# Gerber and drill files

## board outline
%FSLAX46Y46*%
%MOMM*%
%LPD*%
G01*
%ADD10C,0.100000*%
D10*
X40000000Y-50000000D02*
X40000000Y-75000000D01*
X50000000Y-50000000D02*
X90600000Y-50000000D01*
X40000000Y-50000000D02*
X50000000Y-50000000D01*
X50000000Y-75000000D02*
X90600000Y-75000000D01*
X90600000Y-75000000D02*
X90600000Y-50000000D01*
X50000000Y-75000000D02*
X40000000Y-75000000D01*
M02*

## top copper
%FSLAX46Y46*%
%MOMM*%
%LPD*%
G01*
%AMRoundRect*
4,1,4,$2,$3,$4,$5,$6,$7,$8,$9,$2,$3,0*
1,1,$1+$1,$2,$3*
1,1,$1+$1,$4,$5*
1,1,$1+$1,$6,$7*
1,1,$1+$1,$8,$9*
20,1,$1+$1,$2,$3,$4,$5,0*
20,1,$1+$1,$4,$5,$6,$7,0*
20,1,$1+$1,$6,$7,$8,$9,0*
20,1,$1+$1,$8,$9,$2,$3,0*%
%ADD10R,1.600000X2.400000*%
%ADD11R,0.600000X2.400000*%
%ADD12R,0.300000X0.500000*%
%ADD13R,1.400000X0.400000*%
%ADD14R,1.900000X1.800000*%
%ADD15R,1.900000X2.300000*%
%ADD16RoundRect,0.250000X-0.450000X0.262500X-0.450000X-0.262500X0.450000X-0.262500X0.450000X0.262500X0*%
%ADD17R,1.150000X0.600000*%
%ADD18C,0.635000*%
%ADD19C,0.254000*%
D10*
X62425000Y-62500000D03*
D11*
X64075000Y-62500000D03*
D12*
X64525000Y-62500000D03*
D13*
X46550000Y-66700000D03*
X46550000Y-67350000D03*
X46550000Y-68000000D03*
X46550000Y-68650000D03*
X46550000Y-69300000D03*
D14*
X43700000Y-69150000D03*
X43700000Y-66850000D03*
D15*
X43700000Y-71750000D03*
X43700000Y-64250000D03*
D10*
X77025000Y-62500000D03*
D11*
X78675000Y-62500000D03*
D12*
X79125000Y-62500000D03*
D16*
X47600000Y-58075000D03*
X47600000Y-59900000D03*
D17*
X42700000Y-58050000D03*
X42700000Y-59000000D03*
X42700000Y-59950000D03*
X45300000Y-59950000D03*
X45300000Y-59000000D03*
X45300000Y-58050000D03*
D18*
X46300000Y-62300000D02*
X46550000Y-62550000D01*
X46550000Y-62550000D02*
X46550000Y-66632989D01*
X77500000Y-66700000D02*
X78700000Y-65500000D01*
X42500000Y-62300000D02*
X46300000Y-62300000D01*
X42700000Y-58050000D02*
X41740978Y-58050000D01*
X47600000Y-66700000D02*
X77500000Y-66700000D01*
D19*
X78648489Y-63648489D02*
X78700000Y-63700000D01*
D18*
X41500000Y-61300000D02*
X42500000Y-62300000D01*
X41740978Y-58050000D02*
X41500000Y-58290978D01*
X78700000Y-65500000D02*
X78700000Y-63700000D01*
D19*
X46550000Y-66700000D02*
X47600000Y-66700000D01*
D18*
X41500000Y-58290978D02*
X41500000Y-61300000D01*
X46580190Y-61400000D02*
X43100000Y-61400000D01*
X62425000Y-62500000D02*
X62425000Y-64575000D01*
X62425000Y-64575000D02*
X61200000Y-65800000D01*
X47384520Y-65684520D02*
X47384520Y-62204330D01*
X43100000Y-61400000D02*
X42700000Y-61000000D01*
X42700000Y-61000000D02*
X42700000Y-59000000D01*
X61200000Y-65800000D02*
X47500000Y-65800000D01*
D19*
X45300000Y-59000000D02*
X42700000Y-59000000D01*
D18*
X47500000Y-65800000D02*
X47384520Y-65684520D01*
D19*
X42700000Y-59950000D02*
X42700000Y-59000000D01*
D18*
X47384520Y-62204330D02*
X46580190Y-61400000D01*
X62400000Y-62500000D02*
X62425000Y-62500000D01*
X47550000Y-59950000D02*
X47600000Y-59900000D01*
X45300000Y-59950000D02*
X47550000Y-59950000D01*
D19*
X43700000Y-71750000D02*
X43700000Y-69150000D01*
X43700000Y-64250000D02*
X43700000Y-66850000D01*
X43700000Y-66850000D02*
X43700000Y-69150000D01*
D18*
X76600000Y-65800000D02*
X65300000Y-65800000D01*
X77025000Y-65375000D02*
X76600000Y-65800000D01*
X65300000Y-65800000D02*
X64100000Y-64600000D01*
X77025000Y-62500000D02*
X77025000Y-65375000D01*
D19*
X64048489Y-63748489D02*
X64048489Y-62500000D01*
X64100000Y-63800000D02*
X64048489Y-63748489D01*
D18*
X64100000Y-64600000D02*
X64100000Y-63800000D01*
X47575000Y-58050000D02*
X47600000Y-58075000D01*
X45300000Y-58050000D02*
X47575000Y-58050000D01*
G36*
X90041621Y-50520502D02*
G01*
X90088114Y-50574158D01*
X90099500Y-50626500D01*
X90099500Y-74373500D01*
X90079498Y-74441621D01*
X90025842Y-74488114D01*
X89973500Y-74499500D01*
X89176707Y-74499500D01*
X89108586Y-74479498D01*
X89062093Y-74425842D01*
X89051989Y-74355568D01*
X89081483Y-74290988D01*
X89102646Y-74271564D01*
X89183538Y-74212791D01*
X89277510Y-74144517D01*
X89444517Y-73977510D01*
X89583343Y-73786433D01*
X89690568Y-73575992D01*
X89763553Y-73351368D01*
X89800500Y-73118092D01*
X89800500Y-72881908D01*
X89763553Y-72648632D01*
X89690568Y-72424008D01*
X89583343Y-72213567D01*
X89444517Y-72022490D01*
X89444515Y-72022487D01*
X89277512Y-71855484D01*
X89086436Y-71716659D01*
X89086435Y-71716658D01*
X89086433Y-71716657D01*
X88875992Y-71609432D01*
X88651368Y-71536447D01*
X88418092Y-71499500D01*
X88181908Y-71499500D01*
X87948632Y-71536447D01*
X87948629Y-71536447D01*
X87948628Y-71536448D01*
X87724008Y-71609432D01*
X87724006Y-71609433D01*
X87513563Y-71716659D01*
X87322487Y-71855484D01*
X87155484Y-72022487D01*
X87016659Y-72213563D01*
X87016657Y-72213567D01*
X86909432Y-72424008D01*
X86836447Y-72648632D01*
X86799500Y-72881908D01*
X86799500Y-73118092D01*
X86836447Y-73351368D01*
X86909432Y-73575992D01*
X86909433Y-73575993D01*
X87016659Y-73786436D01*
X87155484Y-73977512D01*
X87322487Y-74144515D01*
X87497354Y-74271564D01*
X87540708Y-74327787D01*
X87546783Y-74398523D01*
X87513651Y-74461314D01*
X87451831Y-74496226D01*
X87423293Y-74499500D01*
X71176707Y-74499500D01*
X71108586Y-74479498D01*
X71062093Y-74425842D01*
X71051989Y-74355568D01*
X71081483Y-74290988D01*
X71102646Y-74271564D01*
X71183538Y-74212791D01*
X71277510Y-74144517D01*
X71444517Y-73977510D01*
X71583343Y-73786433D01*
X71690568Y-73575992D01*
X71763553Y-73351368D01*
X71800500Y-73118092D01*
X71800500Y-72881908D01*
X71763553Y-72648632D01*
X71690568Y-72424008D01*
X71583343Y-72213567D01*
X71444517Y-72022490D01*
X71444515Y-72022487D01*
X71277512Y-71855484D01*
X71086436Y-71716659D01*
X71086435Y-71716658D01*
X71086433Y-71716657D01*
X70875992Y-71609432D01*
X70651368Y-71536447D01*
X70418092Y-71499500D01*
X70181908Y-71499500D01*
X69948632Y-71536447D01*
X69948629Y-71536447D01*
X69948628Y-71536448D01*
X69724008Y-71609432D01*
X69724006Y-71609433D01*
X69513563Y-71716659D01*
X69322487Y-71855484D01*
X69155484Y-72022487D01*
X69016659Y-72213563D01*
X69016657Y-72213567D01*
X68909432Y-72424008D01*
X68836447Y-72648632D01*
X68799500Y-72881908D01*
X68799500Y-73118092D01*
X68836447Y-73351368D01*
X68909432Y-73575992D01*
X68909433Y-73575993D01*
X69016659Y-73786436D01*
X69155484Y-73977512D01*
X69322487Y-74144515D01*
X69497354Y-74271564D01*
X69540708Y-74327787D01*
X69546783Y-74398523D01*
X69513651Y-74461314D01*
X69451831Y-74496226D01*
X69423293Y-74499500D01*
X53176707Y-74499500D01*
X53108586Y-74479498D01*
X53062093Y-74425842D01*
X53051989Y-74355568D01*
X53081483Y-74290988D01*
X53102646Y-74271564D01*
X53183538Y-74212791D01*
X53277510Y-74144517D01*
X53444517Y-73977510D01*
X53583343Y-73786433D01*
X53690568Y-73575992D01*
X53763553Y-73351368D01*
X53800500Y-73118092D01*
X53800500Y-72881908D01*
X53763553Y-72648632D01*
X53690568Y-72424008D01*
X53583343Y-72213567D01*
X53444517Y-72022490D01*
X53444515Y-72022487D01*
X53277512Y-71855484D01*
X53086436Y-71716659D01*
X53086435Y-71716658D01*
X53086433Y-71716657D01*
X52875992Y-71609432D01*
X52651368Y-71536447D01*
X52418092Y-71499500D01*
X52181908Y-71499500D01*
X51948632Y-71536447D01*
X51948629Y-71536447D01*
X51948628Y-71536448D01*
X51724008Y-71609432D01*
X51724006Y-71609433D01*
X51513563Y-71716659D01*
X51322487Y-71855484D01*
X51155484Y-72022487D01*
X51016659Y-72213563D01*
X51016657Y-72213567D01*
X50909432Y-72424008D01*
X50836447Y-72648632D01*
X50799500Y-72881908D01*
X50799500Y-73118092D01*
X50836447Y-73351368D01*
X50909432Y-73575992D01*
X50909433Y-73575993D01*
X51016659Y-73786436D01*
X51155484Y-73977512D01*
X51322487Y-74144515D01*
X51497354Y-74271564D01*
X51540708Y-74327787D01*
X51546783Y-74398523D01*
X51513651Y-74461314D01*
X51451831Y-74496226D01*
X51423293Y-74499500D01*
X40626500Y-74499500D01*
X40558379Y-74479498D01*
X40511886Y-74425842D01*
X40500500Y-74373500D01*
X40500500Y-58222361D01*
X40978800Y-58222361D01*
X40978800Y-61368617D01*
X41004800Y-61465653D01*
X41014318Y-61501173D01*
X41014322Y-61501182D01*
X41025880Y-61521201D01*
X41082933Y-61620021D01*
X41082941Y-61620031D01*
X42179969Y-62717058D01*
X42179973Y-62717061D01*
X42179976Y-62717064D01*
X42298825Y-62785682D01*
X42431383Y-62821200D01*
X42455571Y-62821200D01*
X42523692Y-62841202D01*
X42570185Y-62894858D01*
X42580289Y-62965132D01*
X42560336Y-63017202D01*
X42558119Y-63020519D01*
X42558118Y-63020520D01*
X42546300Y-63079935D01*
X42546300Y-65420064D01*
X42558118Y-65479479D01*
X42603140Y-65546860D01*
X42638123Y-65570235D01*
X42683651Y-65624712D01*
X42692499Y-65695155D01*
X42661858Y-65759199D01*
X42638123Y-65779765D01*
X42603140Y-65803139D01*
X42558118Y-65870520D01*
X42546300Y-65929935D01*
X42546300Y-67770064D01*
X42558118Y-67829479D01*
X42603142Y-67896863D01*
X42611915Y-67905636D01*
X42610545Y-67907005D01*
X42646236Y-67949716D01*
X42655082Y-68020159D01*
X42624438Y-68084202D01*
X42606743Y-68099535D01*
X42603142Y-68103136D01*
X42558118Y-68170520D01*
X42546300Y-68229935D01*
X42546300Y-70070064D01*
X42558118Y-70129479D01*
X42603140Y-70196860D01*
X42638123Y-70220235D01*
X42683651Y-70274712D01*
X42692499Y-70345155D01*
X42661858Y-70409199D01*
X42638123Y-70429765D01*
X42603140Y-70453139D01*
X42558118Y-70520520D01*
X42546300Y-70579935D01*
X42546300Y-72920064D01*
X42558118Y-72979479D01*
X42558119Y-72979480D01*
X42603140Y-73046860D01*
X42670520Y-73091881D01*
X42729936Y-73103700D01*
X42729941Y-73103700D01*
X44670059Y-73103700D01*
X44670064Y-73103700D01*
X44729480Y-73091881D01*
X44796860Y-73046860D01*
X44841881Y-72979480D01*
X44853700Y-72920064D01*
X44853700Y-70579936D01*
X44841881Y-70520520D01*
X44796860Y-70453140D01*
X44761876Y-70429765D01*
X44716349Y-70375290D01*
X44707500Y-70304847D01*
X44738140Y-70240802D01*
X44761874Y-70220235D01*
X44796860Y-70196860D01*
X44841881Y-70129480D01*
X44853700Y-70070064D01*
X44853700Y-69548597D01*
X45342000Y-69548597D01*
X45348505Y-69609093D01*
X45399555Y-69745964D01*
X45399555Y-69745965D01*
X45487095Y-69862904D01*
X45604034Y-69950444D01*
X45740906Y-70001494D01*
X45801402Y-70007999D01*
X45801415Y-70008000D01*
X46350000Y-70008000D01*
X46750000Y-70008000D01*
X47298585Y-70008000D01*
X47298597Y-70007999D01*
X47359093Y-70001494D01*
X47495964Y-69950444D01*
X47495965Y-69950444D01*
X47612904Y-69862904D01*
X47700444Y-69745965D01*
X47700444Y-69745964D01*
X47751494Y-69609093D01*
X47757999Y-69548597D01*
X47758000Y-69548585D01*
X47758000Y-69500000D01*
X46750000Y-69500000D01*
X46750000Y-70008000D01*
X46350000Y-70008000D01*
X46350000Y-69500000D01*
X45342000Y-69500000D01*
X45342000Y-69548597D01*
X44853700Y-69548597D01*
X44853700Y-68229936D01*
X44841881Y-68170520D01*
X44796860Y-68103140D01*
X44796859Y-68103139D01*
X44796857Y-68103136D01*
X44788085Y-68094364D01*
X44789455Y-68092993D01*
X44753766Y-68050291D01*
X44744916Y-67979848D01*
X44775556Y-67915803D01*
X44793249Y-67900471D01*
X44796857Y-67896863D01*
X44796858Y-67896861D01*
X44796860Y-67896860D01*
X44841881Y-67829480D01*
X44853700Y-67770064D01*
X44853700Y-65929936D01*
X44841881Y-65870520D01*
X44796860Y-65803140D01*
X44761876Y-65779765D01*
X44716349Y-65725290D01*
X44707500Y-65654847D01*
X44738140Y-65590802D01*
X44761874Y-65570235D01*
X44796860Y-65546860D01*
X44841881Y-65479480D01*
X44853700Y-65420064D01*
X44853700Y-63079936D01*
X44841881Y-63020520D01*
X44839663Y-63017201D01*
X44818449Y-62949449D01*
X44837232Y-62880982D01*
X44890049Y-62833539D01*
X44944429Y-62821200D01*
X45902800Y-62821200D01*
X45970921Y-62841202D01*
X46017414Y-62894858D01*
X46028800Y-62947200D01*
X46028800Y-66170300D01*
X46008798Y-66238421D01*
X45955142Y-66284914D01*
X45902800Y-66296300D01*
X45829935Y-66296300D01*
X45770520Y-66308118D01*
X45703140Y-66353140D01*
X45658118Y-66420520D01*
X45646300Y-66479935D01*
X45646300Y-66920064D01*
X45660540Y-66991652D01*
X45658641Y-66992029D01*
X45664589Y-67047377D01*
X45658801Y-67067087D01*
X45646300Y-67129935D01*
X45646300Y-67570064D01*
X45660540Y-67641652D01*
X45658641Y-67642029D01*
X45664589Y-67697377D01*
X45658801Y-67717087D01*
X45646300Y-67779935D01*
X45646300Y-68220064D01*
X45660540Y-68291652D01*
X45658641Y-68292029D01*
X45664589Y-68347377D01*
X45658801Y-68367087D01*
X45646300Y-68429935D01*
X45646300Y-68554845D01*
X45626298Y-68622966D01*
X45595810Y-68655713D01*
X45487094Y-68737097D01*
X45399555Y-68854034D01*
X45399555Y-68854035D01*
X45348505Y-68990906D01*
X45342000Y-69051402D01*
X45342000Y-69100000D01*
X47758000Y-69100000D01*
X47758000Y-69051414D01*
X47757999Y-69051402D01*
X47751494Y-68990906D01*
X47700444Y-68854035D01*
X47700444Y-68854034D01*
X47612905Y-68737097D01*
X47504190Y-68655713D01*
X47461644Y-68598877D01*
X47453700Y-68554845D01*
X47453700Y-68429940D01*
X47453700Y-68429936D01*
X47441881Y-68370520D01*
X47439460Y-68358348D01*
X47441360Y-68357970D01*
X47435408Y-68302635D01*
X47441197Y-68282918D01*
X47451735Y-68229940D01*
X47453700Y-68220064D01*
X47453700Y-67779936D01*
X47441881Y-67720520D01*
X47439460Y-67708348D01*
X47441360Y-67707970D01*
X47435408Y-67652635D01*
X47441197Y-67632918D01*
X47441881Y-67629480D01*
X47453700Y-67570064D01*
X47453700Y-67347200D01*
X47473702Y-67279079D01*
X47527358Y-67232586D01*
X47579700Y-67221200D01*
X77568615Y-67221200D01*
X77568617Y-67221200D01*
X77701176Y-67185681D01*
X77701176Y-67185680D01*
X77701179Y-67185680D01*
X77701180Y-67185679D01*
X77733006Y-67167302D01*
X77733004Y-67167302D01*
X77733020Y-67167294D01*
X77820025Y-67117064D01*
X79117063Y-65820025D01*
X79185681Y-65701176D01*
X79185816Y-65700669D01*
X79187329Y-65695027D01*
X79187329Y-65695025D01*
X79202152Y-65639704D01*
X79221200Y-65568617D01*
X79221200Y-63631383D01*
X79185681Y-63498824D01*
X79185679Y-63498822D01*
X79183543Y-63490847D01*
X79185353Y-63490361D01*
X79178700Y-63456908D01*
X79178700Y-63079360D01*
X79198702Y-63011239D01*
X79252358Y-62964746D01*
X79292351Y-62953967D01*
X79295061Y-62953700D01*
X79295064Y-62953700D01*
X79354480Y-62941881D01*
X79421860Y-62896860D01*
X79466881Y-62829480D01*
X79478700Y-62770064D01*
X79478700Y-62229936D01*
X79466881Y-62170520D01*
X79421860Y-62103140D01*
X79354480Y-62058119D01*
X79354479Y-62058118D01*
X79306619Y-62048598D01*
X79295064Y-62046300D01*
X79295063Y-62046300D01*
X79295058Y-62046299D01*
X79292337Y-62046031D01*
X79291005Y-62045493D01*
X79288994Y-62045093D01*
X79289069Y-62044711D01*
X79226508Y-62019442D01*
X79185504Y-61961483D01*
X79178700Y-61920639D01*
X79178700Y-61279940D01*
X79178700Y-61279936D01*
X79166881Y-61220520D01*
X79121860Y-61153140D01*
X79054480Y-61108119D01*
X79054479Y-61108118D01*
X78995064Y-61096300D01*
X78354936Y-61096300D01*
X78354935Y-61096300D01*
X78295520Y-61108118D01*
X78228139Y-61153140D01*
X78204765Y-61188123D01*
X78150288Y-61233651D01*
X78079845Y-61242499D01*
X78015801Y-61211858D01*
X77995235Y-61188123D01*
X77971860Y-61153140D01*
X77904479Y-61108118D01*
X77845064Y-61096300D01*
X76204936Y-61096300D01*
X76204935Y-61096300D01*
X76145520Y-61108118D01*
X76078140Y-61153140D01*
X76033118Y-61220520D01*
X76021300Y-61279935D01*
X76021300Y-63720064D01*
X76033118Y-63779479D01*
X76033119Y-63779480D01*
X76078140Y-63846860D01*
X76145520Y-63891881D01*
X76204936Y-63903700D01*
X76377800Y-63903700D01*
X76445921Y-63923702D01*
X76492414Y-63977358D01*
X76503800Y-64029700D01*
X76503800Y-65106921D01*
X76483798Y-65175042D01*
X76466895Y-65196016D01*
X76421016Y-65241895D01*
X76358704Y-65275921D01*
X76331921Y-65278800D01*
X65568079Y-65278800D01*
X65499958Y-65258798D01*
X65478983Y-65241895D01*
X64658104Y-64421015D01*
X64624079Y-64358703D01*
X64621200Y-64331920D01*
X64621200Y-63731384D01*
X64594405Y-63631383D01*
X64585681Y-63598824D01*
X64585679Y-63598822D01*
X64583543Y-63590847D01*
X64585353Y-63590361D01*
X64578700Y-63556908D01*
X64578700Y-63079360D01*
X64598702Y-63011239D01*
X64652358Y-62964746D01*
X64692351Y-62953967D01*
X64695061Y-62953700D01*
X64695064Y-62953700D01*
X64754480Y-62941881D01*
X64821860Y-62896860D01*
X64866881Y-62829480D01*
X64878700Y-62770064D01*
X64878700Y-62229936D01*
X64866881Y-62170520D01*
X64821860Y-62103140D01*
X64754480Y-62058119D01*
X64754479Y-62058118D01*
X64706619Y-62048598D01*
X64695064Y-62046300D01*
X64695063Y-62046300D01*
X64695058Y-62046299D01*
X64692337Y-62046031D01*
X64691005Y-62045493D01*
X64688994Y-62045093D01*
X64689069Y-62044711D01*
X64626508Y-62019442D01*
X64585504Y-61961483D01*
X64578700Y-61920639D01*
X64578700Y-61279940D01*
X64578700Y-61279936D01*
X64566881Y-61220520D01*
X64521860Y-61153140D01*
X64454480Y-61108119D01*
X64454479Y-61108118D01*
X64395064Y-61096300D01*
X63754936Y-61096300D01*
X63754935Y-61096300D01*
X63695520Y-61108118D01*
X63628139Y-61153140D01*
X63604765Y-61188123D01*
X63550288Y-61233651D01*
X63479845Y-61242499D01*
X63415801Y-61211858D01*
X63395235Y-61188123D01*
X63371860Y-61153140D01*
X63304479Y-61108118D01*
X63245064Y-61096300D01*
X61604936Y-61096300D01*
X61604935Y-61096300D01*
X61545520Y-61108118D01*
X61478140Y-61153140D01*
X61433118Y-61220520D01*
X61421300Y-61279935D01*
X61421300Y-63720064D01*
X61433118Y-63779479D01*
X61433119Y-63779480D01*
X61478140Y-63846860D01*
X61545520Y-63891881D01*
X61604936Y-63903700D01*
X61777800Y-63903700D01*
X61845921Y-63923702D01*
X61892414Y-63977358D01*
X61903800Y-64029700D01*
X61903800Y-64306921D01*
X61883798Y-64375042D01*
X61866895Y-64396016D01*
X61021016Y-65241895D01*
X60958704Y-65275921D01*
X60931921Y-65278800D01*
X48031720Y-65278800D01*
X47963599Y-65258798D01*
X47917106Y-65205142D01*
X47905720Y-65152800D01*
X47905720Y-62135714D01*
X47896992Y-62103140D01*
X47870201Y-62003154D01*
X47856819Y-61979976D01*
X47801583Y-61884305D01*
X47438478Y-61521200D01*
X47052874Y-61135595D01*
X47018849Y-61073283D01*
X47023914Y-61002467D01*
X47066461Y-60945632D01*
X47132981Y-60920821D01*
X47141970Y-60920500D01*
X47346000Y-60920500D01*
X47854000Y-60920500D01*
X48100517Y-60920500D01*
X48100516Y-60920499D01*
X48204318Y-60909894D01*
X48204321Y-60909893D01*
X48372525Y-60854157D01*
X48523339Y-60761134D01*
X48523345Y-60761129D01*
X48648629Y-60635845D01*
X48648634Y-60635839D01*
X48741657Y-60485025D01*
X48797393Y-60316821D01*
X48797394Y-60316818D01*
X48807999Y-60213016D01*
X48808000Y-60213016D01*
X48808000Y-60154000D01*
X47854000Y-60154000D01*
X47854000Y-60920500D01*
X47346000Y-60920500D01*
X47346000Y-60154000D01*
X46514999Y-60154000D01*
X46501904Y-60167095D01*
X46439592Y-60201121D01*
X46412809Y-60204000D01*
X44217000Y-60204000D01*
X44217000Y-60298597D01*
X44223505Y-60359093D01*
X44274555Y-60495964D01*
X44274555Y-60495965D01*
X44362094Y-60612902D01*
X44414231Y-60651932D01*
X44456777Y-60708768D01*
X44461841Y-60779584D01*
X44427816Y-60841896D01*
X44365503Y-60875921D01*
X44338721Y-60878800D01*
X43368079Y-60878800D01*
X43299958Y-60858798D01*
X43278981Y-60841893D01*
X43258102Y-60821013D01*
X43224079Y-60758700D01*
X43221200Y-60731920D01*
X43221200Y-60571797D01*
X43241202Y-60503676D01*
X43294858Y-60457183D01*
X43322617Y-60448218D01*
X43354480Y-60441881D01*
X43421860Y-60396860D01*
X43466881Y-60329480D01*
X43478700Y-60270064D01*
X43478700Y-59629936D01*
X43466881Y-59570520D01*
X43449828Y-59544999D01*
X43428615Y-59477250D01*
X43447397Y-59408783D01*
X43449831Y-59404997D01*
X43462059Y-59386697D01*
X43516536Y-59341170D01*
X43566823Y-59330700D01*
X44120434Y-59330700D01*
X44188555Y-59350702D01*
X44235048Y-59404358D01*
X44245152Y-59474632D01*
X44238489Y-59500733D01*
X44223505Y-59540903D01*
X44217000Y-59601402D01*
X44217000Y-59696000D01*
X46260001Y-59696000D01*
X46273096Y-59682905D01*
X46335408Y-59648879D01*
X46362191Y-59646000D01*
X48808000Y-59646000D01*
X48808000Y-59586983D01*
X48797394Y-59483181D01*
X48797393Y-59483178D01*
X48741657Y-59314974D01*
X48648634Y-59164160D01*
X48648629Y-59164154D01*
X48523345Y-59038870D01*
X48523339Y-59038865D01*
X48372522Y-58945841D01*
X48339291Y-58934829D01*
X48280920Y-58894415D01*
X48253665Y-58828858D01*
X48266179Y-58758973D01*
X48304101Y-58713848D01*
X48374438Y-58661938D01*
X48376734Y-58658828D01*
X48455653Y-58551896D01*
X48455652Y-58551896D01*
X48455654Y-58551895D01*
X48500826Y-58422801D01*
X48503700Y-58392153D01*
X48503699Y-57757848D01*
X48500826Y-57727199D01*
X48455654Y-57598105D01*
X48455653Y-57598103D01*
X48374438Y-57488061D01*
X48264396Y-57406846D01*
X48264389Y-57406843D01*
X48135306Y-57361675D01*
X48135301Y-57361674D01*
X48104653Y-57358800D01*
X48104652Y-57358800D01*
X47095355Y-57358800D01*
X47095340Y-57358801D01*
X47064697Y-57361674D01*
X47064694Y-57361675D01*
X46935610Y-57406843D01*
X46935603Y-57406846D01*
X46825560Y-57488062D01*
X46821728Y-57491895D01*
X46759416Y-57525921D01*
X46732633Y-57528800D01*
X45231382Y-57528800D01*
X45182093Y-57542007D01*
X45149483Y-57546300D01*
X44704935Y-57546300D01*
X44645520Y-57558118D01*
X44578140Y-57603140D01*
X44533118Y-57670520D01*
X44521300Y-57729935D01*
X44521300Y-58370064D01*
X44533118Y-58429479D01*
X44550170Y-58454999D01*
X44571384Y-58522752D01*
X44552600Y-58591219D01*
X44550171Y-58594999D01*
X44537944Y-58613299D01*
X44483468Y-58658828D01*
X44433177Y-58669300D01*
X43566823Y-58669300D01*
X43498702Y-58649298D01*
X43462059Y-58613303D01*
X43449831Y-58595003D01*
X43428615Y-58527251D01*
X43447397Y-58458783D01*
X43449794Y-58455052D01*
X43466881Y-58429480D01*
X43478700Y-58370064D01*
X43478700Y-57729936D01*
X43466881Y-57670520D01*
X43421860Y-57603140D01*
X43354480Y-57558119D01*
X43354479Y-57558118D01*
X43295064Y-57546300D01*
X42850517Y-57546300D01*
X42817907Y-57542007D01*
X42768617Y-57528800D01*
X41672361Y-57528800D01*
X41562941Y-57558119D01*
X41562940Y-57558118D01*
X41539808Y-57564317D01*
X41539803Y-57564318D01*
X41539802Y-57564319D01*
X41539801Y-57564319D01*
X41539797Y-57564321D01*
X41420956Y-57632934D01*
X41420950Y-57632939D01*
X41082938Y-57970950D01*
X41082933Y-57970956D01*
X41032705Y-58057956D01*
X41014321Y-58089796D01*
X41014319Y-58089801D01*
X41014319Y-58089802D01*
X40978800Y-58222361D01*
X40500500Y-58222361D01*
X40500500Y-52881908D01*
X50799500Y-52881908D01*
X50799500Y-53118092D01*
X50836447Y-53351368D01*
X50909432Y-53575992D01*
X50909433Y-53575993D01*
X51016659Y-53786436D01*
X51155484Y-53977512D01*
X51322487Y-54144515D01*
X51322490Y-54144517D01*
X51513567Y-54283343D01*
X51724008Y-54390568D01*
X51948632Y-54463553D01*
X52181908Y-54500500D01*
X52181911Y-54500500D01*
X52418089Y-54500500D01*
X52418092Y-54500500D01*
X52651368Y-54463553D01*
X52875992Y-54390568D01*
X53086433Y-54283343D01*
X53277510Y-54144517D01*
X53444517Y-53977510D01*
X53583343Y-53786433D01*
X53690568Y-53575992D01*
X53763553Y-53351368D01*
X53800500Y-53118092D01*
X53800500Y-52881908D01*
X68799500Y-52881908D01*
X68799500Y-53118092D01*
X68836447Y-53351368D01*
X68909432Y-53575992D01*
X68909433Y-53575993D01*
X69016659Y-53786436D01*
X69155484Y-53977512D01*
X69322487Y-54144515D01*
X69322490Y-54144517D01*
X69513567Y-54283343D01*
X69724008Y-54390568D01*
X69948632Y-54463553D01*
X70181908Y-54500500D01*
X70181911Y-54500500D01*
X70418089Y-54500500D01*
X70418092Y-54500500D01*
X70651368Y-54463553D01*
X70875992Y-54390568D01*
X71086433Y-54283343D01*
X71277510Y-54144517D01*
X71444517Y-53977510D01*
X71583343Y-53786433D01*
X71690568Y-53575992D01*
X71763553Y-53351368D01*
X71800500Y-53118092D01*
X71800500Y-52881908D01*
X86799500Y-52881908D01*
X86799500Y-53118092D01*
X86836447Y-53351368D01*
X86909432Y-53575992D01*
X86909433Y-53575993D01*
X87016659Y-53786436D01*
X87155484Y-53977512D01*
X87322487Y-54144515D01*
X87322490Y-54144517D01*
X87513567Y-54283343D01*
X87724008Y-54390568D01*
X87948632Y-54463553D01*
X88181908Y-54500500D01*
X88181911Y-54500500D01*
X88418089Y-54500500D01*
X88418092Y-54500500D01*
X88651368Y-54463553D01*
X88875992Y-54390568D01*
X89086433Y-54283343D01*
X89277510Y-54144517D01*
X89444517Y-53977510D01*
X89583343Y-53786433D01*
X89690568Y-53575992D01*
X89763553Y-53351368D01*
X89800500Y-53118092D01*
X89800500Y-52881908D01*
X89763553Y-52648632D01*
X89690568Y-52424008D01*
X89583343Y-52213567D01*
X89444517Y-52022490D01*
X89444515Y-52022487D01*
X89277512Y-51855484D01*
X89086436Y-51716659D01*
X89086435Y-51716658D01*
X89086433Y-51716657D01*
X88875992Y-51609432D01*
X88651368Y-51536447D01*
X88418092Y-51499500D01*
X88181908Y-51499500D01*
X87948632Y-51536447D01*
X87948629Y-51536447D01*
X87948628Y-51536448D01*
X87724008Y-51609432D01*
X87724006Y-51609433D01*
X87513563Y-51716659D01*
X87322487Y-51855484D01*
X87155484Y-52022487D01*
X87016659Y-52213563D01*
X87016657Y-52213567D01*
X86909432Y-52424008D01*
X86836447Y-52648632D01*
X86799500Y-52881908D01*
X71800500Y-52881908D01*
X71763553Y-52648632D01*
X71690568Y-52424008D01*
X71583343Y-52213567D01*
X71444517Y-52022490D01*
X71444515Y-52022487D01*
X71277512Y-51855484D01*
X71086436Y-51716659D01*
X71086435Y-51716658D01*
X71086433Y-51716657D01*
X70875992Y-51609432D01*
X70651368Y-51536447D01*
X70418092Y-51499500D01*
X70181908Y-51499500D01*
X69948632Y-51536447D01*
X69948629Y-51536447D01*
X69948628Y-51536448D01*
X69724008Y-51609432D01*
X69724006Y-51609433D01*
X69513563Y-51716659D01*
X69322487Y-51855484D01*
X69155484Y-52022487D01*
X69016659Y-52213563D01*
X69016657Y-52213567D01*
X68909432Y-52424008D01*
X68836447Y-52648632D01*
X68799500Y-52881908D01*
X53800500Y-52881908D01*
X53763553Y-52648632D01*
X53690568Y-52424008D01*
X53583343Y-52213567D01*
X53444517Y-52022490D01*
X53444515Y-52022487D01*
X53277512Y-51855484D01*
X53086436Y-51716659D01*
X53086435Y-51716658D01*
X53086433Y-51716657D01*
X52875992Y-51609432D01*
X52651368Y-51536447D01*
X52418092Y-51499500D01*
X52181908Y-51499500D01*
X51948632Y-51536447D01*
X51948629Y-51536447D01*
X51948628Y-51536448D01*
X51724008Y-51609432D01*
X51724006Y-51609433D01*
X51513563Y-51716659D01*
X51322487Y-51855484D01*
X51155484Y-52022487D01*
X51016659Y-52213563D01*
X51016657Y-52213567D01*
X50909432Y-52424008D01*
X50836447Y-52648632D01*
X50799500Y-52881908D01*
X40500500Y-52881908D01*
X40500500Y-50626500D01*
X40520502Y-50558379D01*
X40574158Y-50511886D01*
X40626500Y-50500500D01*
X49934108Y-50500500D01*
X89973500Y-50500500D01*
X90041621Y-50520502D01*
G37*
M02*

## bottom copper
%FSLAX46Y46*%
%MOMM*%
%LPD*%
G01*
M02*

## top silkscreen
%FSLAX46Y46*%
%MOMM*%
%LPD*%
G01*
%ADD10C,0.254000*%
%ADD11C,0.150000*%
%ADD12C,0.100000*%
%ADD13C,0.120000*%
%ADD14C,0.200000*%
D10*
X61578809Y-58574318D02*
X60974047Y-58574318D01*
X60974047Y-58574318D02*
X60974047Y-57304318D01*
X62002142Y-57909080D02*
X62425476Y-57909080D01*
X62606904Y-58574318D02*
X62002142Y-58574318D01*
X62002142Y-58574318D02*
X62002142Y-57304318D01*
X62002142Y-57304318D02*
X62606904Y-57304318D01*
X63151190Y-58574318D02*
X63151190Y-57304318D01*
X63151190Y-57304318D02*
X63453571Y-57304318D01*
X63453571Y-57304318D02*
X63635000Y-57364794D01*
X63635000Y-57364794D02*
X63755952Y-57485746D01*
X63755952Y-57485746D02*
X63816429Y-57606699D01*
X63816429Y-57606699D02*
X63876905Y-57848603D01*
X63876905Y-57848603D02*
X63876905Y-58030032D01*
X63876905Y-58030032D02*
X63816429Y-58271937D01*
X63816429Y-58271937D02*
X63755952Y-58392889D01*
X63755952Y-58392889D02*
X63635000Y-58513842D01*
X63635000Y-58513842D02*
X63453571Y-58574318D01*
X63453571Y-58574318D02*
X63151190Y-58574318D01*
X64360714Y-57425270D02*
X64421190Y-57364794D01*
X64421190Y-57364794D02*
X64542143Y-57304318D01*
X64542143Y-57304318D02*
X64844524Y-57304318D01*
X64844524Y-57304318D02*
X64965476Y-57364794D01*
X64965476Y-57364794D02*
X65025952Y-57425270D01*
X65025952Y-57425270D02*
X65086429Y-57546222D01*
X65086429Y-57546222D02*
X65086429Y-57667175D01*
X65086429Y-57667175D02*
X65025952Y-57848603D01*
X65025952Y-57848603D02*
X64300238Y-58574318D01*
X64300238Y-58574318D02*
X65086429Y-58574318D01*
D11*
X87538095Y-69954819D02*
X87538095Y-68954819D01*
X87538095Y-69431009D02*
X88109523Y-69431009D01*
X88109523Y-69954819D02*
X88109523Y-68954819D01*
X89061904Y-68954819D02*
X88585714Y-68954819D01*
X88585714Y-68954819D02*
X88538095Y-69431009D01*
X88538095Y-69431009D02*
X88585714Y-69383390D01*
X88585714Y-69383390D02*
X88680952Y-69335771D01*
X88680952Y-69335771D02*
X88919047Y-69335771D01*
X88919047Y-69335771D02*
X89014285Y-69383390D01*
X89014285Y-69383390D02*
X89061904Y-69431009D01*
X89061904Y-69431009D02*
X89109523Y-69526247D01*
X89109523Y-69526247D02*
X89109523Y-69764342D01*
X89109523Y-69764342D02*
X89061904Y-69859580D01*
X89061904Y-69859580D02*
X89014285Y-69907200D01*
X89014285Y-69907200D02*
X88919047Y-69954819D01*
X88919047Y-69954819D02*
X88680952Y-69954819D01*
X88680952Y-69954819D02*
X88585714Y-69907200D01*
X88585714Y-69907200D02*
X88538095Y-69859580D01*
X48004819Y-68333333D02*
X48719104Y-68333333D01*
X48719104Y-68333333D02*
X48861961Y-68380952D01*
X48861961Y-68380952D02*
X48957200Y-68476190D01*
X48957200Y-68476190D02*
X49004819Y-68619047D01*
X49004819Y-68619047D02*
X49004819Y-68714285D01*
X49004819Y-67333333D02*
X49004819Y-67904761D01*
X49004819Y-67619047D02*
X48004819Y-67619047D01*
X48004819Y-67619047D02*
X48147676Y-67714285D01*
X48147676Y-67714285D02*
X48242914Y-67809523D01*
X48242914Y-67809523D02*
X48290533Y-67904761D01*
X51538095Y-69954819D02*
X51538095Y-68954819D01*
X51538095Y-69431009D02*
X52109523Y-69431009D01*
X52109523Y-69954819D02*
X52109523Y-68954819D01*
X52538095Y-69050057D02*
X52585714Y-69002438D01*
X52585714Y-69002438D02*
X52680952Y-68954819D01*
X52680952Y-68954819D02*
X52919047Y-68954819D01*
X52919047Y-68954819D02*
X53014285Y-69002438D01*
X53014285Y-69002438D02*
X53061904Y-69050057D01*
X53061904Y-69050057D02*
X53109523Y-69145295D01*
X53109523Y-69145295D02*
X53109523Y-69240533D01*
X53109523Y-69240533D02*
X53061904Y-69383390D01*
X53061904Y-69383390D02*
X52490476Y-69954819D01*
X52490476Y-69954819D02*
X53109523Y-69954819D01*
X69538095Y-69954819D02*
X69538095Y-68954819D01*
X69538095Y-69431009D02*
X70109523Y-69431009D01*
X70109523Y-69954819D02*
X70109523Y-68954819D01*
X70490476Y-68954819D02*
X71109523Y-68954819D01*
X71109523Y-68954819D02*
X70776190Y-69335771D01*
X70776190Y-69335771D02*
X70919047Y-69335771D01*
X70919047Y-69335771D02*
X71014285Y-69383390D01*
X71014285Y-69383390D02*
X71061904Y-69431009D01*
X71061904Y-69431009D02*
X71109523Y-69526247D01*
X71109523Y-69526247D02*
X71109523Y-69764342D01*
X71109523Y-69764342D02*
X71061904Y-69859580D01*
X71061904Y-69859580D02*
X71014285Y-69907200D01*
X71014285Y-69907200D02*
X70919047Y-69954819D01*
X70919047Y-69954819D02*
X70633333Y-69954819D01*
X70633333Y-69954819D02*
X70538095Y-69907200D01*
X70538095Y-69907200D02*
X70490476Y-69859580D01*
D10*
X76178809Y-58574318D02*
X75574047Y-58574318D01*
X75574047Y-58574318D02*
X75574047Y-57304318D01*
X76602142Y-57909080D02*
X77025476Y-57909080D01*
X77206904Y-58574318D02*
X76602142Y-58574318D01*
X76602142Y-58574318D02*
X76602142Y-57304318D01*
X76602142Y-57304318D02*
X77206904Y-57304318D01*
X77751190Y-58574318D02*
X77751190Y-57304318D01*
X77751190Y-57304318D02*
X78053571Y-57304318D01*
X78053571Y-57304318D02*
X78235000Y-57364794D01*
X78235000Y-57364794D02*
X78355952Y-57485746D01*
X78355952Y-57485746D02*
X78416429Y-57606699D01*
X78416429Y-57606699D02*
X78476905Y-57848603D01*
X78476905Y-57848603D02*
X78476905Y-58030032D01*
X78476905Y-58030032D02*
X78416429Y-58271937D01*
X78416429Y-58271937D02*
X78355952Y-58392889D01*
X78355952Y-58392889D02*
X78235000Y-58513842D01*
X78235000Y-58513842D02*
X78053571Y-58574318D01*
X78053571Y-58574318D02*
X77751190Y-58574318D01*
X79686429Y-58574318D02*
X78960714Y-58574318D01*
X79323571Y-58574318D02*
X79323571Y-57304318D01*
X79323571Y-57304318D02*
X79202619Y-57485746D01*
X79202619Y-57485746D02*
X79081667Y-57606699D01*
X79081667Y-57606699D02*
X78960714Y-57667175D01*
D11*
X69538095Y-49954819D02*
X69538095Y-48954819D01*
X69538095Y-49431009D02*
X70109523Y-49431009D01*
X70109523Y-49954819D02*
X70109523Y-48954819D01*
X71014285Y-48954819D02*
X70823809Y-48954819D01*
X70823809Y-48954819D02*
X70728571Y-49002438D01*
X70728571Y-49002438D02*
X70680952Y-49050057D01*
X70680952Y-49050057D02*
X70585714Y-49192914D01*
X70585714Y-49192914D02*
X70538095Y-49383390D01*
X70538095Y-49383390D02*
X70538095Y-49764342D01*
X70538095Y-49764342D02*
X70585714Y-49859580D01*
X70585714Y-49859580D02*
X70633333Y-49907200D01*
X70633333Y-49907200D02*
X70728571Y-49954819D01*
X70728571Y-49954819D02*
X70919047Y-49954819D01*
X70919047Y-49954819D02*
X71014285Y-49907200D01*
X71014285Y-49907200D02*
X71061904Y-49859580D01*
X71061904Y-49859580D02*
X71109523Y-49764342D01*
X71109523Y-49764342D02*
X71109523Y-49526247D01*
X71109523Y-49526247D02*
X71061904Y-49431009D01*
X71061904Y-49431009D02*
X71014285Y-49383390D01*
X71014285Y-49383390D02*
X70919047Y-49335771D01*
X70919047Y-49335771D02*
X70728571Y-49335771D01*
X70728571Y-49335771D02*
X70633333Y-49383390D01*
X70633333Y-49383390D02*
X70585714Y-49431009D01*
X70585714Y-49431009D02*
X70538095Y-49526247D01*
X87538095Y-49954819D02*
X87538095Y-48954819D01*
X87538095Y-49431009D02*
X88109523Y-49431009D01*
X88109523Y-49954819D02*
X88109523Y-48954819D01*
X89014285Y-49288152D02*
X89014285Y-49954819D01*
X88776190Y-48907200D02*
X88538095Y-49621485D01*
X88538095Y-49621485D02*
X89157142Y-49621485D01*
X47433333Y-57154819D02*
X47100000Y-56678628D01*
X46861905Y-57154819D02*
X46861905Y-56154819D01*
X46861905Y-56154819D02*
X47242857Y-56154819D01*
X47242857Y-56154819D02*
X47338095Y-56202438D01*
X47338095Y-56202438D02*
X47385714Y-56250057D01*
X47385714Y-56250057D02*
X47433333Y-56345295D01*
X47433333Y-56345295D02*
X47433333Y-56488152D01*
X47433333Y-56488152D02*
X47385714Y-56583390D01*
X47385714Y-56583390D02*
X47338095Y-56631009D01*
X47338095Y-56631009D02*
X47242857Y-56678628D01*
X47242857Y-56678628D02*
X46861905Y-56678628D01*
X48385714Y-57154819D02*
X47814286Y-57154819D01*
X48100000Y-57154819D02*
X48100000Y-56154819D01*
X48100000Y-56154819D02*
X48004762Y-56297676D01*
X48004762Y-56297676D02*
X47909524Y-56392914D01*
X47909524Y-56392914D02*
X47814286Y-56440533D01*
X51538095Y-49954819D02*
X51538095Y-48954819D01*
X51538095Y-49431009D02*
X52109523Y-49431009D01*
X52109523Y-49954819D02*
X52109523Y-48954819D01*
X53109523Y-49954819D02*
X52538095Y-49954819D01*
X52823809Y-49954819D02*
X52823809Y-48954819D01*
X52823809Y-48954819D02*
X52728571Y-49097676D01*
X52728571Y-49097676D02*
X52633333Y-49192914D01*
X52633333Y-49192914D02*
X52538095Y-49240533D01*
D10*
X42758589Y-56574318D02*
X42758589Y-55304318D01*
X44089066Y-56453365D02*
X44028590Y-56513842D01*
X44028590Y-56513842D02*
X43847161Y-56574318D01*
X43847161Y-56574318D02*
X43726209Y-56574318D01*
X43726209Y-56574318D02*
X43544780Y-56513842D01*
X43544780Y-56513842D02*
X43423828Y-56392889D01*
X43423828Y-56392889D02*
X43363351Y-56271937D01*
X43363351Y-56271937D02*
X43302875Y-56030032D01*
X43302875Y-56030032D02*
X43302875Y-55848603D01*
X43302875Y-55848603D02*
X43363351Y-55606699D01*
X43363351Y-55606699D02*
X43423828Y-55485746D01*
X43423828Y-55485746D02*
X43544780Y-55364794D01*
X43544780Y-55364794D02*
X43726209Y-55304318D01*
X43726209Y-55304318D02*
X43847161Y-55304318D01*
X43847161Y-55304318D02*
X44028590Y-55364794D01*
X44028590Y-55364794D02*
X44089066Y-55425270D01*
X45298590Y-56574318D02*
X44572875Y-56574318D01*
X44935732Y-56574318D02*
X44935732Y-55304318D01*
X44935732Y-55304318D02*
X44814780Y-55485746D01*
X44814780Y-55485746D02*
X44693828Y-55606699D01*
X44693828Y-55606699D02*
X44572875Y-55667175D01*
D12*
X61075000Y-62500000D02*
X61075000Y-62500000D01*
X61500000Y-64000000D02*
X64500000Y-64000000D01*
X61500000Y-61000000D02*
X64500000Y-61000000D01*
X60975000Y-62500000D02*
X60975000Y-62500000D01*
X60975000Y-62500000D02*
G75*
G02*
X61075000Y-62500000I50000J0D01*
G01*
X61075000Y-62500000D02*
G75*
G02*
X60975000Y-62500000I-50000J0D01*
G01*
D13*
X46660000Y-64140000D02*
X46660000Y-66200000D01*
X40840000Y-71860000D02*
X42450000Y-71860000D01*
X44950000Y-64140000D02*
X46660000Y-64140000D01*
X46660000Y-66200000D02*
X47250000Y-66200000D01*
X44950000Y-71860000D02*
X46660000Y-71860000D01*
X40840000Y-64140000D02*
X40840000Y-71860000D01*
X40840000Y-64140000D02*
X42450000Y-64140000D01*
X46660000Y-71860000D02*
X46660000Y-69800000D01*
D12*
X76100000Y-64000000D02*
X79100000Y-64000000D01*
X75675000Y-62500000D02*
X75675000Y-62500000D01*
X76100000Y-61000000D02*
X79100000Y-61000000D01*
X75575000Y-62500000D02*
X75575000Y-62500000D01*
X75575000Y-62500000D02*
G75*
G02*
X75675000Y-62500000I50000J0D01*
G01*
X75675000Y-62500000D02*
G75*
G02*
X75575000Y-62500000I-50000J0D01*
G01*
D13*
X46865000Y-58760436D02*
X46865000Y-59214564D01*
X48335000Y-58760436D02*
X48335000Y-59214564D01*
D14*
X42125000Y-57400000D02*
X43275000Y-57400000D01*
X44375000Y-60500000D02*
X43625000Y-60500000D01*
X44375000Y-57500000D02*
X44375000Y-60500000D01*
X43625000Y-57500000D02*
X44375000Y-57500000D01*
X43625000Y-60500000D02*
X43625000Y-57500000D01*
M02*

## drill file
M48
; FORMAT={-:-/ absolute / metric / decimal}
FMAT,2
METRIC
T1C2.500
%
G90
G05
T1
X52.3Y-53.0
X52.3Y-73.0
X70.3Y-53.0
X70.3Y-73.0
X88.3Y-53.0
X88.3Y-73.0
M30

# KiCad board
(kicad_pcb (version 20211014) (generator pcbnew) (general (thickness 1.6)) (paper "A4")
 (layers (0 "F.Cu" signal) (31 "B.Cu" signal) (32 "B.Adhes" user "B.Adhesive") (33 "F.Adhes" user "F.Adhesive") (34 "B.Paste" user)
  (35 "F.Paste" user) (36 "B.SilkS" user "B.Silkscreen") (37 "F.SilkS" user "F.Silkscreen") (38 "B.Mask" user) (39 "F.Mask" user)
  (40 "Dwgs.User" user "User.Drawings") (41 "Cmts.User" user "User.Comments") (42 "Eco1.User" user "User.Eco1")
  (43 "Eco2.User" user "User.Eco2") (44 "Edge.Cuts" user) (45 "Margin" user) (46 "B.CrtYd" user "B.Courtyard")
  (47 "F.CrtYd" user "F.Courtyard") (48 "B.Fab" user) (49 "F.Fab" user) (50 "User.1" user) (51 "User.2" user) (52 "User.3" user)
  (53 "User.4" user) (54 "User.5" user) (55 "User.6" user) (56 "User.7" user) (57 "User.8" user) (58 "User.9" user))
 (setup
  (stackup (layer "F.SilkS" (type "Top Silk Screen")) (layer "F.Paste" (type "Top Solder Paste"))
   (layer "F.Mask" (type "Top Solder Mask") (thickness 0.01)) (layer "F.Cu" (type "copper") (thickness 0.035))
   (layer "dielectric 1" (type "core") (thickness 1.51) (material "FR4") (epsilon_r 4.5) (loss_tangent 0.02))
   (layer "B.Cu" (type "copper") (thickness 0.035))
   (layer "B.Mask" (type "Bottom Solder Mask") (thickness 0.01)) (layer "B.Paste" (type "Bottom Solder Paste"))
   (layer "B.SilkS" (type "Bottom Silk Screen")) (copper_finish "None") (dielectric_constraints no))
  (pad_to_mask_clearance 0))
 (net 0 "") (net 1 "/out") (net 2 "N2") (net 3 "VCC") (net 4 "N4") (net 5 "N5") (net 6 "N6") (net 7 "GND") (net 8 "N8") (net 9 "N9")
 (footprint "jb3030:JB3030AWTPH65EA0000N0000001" (layer "F.Cu") (at 63 62.5)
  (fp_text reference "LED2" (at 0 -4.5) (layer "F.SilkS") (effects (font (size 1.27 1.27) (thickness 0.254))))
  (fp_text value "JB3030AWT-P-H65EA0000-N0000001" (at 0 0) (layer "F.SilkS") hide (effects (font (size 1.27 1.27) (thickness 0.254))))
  (fp_line (start -1.925 0) (end -1.925 0) (layer "F.SilkS") (width 0.1))
  (fp_line (start -1.5 1.5) (end 1.5 1.5) (layer "F.SilkS") (width 0.1))
  (fp_line (start -1.5 -1.5) (end 1.5 -1.5) (layer "F.SilkS") (width 0.1))
  (fp_line (start -2.025 0) (end -2.025 0) (layer "F.SilkS") (width 0.1))
  (fp_arc (start -2.025 0) (mid -1.975 -0.05) (end -1.925 0) (layer "F.SilkS") (width 0.1))
  (fp_arc (start -1.925 0) (mid -1.975 0.05) (end -2.025 0) (layer "F.SilkS") (width 0.1))
  (pad "1" smd rect locked (at -0.575 0) (size 1.6 2.4) (layers "F.Cu" "F.Paste" "F.Mask") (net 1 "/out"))
  (pad "2" smd rect locked (at 1.075 0) (size 0.6 2.4) (layers "F.Cu" "F.Paste" "F.Mask") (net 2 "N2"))
  (pad "3" smd rect locked (at 1.525 0) (size 0.3 0.5) (layers "F.Cu" "F.Paste" "F.Mask")))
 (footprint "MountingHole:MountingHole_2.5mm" (layer "F.Cu") (at 88.3 73)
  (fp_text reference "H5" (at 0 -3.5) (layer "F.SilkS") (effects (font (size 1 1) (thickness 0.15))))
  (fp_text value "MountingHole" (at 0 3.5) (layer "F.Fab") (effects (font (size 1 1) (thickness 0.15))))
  (pad "" np_thru_hole circle (at 0 0) (size 2.5 2.5) (drill 2.5) (layers *.Cu *.Mask)))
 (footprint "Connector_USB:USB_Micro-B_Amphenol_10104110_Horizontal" (layer "F.Cu") (at 45 68 -90)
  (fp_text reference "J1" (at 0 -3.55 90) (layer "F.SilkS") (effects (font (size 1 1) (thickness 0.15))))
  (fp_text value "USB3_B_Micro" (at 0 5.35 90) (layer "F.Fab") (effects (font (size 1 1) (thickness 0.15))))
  (fp_line (start -3.86 -1.66) (end -1.8 -1.66) (layer "F.SilkS") (width 0.12))
  (fp_line (start 3.86 4.16) (end 3.86 2.55) (layer "F.SilkS") (width 0.12))
  (fp_line (start -3.86 0.05) (end -3.86 -1.66) (layer "F.SilkS") (width 0.12))
  (fp_line (start -1.8 -1.66) (end -1.8 -2.25) (layer "F.SilkS") (width 0.12))
  (fp_line (start 3.86 0.05) (end 3.86 -1.66) (layer "F.SilkS") (width 0.12))
  (fp_line (start -3.86 4.16) (end 3.86 4.16) (layer "F.SilkS") (width 0.12))
  (fp_line (start -3.86 4.16) (end -3.86 2.55) (layer "F.SilkS") (width 0.12))
  (fp_line (start 3.86 -1.66) (end 1.8 -1.66) (layer "F.SilkS") (width 0.12))
  (pad "1" smd rect (at -1.3 -1.55 270) (size 0.4 1.4) (layers "F.Cu" "F.Paste" "F.Mask") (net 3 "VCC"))
  (pad "2" smd rect (at -0.65 -1.55 270) (size 0.4 1.4) (layers "F.Cu" "F.Paste" "F.Mask") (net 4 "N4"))
  (pad "3" smd rect (at 0 -1.55 270) (size 0.4 1.4) (layers "F.Cu" "F.Paste" "F.Mask") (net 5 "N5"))
  (pad "4" smd rect (at 0.65 -1.55 270) (size 0.4 1.4) (layers "F.Cu" "F.Paste" "F.Mask") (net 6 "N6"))
  (pad "5" smd rect (at 1.3 -1.55 270) (size 0.4 1.4) (layers "F.Cu" "F.Paste" "F.Mask") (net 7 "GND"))
  (pad "6" smd rect (at 1.15 1.3 270) (size 1.8 1.9) (layers "F.Cu" "F.Paste" "F.Mask") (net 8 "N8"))
  (pad "6" smd rect (at -1.15 1.3 270) (size 1.8 1.9) (layers "F.Cu" "F.Paste" "F.Mask") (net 8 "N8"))
  (pad "6" smd rect (at 3.75 1.3 270) (size 2.3 1.9) (layers "F.Cu" "F.Paste" "F.Mask") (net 8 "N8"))
  (pad "6" smd rect (at -3.75 1.3 270) (size 2.3 1.9) (layers "F.Cu" "F.Paste" "F.Mask") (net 8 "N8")))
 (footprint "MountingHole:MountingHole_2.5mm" (layer "F.Cu") (at 52.3 73)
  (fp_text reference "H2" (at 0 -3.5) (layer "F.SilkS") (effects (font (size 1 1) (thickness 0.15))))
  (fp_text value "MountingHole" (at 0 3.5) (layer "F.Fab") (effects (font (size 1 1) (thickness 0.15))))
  (pad "" np_thru_hole circle (at 0 0) (size 2.5 2.5) (drill 2.5) (layers *.Cu *.Mask)))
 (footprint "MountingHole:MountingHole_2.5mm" (layer "F.Cu") (at 70.3 73)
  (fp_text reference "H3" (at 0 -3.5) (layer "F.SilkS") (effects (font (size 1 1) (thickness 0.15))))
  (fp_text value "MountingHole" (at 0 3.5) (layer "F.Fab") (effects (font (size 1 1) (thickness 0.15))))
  (pad "" np_thru_hole circle (at 0 0) (size 2.5 2.5) (drill 2.5) (layers *.Cu *.Mask)))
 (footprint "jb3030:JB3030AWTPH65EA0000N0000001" (layer "F.Cu") (at 77.6 62.5)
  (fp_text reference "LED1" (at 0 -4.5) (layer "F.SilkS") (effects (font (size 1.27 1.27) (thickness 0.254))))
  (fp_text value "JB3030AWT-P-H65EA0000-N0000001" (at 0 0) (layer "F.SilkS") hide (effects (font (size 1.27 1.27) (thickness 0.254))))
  (fp_line (start -1.5 1.5) (end 1.5 1.5) (layer "F.SilkS") (width 0.1))
  (fp_line (start -1.925 0) (end -1.925 0) (layer "F.SilkS") (width 0.1))
  (fp_line (start -1.5 -1.5) (end 1.5 -1.5) (layer "F.SilkS") (width 0.1))
  (fp_line (start -2.025 0) (end -2.025 0) (layer "F.SilkS") (width 0.1))
  (fp_arc (start -2.025 0) (mid -1.975 -0.05) (end -1.925 0) (layer "F.SilkS") (width 0.1))
  (fp_arc (start -1.925 0) (mid -1.975 0.05) (end -2.025 0) (layer "F.SilkS") (width 0.1))
  (pad "1" smd rect locked (at -0.575 0) (size 1.6 2.4) (layers "F.Cu" "F.Paste" "F.Mask") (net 2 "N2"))
  (pad "2" smd rect locked (at 1.075 0) (size 0.6 2.4) (layers "F.Cu" "F.Paste" "F.Mask") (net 3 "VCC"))
  (pad "3" smd rect locked (at 1.525 0) (size 0.3 0.5) (layers "F.Cu" "F.Paste" "F.Mask")))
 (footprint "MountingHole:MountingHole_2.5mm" (layer "F.Cu") (at 70.3 53)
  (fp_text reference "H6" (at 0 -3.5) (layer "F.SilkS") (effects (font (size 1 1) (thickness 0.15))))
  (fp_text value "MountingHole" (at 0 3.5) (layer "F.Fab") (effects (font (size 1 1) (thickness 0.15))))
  (pad "" np_thru_hole circle (at 0 0) (size 2.5 2.5) (drill 2.5) (layers *.Cu *.Mask)))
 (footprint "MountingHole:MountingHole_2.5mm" (layer "F.Cu") (at 88.3 53)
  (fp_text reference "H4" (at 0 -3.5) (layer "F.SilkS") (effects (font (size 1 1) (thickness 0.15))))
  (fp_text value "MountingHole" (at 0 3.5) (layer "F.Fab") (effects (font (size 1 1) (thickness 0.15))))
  (pad "" np_thru_hole circle (at 0 0) (size 2.5 2.5) (drill 2.5) (layers *.Cu *.Mask)))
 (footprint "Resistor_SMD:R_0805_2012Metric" (layer "F.Cu") (at 47.6 58.9875 -90)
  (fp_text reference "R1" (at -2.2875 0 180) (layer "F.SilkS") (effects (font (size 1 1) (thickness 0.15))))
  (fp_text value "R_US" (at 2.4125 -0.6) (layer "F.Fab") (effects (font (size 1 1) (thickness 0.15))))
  (fp_line (start -0.227064 0.735) (end 0.227064 0.735) (layer "F.SilkS") (width 0.12))
  (fp_line (start -0.227064 -0.735) (end 0.227064 -0.735) (layer "F.SilkS") (width 0.12))
  (pad "1" smd roundrect (at -0.9125 0 270) (size 1.025 1.4) (layers "F.Cu" "F.Paste" "F.Mask") (roundrect_rratio 0.243902439) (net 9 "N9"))
  (pad "2" smd roundrect (at 0.9125 0 270) (size 1.025 1.4) (layers "F.Cu" "F.Paste" "F.Mask") (roundrect_rratio 0.243902439) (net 7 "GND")))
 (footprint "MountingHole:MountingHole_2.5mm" (layer "F.Cu") (at 52.3 53)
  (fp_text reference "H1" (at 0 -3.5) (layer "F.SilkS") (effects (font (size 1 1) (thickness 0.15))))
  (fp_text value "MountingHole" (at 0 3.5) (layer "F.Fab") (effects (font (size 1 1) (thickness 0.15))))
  (pad "" np_thru_hole circle (at 0 0) (size 2.5 2.5) (drill 2.5) (layers *.Cu *.Mask)))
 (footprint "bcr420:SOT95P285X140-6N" (layer "F.Cu") (at 44 59)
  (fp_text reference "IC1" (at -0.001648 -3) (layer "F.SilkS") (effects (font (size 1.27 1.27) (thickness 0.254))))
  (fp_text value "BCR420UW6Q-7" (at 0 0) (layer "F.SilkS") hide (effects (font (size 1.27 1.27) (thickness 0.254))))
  (fp_line (start -1.875 -1.6) (end -0.725 -1.6) (layer "F.SilkS") (width 0.2))
  (fp_line (start 0.375 1.5) (end -0.375 1.5) (layer "F.SilkS") (width 0.2))
  (fp_line (start 0.375 -1.5) (end 0.375 1.5) (layer "F.SilkS") (width 0.2))
  (fp_line (start -0.375 -1.5) (end 0.375 -1.5) (layer "F.SilkS") (width 0.2))
  (fp_line (start -0.375 1.5) (end -0.375 -1.5) (layer "F.SilkS") (width 0.2))
  (pad "1" smd rect locked (at -1.3 -0.95 90) (size 0.6 1.15) (layers "F.Cu" "F.Paste" "F.Mask") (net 3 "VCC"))
  (pad "2" smd rect locked (at -1.3 0 90) (size 0.6 1.15) (layers "F.Cu" "F.Paste" "F.Mask") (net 1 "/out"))
  (pad "3" smd rect locked (at -1.3 0.95 90) (size 0.6 1.15) (layers "F.Cu" "F.Paste" "F.Mask") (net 1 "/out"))
  (pad "4" smd rect locked (at 1.3 0.95 90) (size 0.6 1.15) (layers "F.Cu" "F.Paste" "F.Mask") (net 7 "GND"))
  (pad "5" smd rect locked (at 1.3 0 90) (size 0.6 1.15) (layers "F.Cu" "F.Paste" "F.Mask") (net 1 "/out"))
  (pad "6" smd rect locked (at 1.3 -0.95 90) (size 0.6 1.15) (layers "F.Cu" "F.Paste" "F.Mask") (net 9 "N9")))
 (gr_line (start 40 50) (end 40 75) (layer "Edge.Cuts") (width 0.1))
 (gr_line (start 50 50) (end 90.6 50) (layer "Edge.Cuts") (width 0.1))
 (gr_line (start 40 50) (end 50 50) (layer "Edge.Cuts") (width 0.1))
 (gr_line (start 50 75) (end 90.6 75) (layer "Edge.Cuts") (width 0.1))
 (gr_line (start 90.6 75) (end 90.6 50) (layer "Edge.Cuts") (width 0.1))
 (gr_line (start 50 75) (end 40 75) (layer "Edge.Cuts") (width 0.1))
 (segment (start 46.3 62.3) (end 46.55 62.55) (width 0.635) (layer "F.Cu") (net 3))
 (segment (start 46.55 62.55) (end 46.55 66.632989) (width 0.635) (layer "F.Cu") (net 3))
 (segment (start 77.5 66.7) (end 78.7 65.5) (width 0.635) (layer "F.Cu") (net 3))
 (segment (start 42.5 62.3) (end 46.3 62.3) (width 0.635) (layer "F.Cu") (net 3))
 (segment (start 42.7 58.05) (end 41.740978 58.05) (width 0.635) (layer "F.Cu") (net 3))
 (segment (start 47.6 66.7) (end 77.5 66.7) (width 0.635) (layer "F.Cu") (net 3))
 (segment (start 78.648489 63.648489) (end 78.7 63.7) (width 0.254) (layer "F.Cu") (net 3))
 (segment (start 41.5 61.3) (end 42.5 62.3) (width 0.635) (layer "F.Cu") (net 3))
 (segment (start 41.740978 58.05) (end 41.5 58.290978) (width 0.635) (layer "F.Cu") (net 3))
 (segment (start 78.7 65.5) (end 78.7 63.7) (width 0.635) (layer "F.Cu") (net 3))
 (segment (start 46.55 66.7) (end 47.6 66.7) (width 0.254) (layer "F.Cu") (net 3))
 (segment (start 41.5 58.290978) (end 41.5 61.3) (width 0.635) (layer "F.Cu") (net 3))
 (segment (start 46.58019 61.4) (end 43.1 61.4) (width 0.635) (layer "F.Cu") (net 1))
 (segment (start 62.425 62.5) (end 62.425 64.575) (width 0.635) (layer "F.Cu") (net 1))
 (segment (start 62.425 64.575) (end 61.2 65.8) (width 0.635) (layer "F.Cu") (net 1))
 (segment (start 47.38452 65.68452) (end 47.38452 62.20433) (width 0.635) (layer "F.Cu") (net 1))
 (segment (start 43.1 61.4) (end 42.7 61) (width 0.635) (layer "F.Cu") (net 1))
 (segment (start 42.7 61) (end 42.7 59) (width 0.635) (layer "F.Cu") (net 1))
 (segment (start 61.2 65.8) (end 47.5 65.8) (width 0.635) (layer "F.Cu") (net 1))
 (segment (start 45.3 59) (end 42.7 59) (width 0.254) (layer "F.Cu") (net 1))
 (segment (start 47.5 65.8) (end 47.38452 65.68452) (width 0.635) (layer "F.Cu") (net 1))
 (segment (start 42.7 59.95) (end 42.7 59) (width 0.254) (layer "F.Cu") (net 1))
 (segment (start 47.38452 62.20433) (end 46.58019 61.4) (width 0.635) (layer "F.Cu") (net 1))
 (segment (start 62.4 62.5) (end 62.425 62.5) (width 0.635) (layer "F.Cu") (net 1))
 (segment (start 47.55 59.95) (end 47.6 59.9) (width 0.635) (layer "F.Cu") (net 7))
 (segment (start 45.3 59.95) (end 47.55 59.95) (width 0.635) (layer "F.Cu") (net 7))
 (segment (start 43.7 71.75) (end 43.7 69.15) (width 0.254) (layer "F.Cu") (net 8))
 (segment (start 43.7 64.25) (end 43.7 66.85) (width 0.254) (layer "F.Cu") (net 8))
 (segment (start 43.7 66.85) (end 43.7 69.15) (width 0.254) (layer "F.Cu") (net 8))
 (segment (start 76.6 65.8) (end 65.3 65.8) (width 0.635) (layer "F.Cu") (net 2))
 (segment (start 77.025 65.375) (end 76.6 65.8) (width 0.635) (layer "F.Cu") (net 2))
 (segment (start 65.3 65.8) (end 64.1 64.6) (width 0.635) (layer "F.Cu") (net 2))
 (segment (start 77.025 62.5) (end 77.025 65.375) (width 0.635) (layer "F.Cu") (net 2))
 (segment (start 64.048489 63.748489) (end 64.048489 62.5) (width 0.254) (layer "F.Cu") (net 2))
 (segment (start 64.1 63.8) (end 64.048489 63.748489) (width 0.254) (layer "F.Cu") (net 2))
 (segment (start 64.1 64.6) (end 64.1 63.8) (width 0.635) (layer "F.Cu") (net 2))
 (segment (start 47.575 58.05) (end 47.6 58.075) (width 0.635) (layer "F.Cu") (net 9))
 (segment (start 45.3 58.05) (end 47.575 58.05) (width 0.635) (layer "F.Cu") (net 9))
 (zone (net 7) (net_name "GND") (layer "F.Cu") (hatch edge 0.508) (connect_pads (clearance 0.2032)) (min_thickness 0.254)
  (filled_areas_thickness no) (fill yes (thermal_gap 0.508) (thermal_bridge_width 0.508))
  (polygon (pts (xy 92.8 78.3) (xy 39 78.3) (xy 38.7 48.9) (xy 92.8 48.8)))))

